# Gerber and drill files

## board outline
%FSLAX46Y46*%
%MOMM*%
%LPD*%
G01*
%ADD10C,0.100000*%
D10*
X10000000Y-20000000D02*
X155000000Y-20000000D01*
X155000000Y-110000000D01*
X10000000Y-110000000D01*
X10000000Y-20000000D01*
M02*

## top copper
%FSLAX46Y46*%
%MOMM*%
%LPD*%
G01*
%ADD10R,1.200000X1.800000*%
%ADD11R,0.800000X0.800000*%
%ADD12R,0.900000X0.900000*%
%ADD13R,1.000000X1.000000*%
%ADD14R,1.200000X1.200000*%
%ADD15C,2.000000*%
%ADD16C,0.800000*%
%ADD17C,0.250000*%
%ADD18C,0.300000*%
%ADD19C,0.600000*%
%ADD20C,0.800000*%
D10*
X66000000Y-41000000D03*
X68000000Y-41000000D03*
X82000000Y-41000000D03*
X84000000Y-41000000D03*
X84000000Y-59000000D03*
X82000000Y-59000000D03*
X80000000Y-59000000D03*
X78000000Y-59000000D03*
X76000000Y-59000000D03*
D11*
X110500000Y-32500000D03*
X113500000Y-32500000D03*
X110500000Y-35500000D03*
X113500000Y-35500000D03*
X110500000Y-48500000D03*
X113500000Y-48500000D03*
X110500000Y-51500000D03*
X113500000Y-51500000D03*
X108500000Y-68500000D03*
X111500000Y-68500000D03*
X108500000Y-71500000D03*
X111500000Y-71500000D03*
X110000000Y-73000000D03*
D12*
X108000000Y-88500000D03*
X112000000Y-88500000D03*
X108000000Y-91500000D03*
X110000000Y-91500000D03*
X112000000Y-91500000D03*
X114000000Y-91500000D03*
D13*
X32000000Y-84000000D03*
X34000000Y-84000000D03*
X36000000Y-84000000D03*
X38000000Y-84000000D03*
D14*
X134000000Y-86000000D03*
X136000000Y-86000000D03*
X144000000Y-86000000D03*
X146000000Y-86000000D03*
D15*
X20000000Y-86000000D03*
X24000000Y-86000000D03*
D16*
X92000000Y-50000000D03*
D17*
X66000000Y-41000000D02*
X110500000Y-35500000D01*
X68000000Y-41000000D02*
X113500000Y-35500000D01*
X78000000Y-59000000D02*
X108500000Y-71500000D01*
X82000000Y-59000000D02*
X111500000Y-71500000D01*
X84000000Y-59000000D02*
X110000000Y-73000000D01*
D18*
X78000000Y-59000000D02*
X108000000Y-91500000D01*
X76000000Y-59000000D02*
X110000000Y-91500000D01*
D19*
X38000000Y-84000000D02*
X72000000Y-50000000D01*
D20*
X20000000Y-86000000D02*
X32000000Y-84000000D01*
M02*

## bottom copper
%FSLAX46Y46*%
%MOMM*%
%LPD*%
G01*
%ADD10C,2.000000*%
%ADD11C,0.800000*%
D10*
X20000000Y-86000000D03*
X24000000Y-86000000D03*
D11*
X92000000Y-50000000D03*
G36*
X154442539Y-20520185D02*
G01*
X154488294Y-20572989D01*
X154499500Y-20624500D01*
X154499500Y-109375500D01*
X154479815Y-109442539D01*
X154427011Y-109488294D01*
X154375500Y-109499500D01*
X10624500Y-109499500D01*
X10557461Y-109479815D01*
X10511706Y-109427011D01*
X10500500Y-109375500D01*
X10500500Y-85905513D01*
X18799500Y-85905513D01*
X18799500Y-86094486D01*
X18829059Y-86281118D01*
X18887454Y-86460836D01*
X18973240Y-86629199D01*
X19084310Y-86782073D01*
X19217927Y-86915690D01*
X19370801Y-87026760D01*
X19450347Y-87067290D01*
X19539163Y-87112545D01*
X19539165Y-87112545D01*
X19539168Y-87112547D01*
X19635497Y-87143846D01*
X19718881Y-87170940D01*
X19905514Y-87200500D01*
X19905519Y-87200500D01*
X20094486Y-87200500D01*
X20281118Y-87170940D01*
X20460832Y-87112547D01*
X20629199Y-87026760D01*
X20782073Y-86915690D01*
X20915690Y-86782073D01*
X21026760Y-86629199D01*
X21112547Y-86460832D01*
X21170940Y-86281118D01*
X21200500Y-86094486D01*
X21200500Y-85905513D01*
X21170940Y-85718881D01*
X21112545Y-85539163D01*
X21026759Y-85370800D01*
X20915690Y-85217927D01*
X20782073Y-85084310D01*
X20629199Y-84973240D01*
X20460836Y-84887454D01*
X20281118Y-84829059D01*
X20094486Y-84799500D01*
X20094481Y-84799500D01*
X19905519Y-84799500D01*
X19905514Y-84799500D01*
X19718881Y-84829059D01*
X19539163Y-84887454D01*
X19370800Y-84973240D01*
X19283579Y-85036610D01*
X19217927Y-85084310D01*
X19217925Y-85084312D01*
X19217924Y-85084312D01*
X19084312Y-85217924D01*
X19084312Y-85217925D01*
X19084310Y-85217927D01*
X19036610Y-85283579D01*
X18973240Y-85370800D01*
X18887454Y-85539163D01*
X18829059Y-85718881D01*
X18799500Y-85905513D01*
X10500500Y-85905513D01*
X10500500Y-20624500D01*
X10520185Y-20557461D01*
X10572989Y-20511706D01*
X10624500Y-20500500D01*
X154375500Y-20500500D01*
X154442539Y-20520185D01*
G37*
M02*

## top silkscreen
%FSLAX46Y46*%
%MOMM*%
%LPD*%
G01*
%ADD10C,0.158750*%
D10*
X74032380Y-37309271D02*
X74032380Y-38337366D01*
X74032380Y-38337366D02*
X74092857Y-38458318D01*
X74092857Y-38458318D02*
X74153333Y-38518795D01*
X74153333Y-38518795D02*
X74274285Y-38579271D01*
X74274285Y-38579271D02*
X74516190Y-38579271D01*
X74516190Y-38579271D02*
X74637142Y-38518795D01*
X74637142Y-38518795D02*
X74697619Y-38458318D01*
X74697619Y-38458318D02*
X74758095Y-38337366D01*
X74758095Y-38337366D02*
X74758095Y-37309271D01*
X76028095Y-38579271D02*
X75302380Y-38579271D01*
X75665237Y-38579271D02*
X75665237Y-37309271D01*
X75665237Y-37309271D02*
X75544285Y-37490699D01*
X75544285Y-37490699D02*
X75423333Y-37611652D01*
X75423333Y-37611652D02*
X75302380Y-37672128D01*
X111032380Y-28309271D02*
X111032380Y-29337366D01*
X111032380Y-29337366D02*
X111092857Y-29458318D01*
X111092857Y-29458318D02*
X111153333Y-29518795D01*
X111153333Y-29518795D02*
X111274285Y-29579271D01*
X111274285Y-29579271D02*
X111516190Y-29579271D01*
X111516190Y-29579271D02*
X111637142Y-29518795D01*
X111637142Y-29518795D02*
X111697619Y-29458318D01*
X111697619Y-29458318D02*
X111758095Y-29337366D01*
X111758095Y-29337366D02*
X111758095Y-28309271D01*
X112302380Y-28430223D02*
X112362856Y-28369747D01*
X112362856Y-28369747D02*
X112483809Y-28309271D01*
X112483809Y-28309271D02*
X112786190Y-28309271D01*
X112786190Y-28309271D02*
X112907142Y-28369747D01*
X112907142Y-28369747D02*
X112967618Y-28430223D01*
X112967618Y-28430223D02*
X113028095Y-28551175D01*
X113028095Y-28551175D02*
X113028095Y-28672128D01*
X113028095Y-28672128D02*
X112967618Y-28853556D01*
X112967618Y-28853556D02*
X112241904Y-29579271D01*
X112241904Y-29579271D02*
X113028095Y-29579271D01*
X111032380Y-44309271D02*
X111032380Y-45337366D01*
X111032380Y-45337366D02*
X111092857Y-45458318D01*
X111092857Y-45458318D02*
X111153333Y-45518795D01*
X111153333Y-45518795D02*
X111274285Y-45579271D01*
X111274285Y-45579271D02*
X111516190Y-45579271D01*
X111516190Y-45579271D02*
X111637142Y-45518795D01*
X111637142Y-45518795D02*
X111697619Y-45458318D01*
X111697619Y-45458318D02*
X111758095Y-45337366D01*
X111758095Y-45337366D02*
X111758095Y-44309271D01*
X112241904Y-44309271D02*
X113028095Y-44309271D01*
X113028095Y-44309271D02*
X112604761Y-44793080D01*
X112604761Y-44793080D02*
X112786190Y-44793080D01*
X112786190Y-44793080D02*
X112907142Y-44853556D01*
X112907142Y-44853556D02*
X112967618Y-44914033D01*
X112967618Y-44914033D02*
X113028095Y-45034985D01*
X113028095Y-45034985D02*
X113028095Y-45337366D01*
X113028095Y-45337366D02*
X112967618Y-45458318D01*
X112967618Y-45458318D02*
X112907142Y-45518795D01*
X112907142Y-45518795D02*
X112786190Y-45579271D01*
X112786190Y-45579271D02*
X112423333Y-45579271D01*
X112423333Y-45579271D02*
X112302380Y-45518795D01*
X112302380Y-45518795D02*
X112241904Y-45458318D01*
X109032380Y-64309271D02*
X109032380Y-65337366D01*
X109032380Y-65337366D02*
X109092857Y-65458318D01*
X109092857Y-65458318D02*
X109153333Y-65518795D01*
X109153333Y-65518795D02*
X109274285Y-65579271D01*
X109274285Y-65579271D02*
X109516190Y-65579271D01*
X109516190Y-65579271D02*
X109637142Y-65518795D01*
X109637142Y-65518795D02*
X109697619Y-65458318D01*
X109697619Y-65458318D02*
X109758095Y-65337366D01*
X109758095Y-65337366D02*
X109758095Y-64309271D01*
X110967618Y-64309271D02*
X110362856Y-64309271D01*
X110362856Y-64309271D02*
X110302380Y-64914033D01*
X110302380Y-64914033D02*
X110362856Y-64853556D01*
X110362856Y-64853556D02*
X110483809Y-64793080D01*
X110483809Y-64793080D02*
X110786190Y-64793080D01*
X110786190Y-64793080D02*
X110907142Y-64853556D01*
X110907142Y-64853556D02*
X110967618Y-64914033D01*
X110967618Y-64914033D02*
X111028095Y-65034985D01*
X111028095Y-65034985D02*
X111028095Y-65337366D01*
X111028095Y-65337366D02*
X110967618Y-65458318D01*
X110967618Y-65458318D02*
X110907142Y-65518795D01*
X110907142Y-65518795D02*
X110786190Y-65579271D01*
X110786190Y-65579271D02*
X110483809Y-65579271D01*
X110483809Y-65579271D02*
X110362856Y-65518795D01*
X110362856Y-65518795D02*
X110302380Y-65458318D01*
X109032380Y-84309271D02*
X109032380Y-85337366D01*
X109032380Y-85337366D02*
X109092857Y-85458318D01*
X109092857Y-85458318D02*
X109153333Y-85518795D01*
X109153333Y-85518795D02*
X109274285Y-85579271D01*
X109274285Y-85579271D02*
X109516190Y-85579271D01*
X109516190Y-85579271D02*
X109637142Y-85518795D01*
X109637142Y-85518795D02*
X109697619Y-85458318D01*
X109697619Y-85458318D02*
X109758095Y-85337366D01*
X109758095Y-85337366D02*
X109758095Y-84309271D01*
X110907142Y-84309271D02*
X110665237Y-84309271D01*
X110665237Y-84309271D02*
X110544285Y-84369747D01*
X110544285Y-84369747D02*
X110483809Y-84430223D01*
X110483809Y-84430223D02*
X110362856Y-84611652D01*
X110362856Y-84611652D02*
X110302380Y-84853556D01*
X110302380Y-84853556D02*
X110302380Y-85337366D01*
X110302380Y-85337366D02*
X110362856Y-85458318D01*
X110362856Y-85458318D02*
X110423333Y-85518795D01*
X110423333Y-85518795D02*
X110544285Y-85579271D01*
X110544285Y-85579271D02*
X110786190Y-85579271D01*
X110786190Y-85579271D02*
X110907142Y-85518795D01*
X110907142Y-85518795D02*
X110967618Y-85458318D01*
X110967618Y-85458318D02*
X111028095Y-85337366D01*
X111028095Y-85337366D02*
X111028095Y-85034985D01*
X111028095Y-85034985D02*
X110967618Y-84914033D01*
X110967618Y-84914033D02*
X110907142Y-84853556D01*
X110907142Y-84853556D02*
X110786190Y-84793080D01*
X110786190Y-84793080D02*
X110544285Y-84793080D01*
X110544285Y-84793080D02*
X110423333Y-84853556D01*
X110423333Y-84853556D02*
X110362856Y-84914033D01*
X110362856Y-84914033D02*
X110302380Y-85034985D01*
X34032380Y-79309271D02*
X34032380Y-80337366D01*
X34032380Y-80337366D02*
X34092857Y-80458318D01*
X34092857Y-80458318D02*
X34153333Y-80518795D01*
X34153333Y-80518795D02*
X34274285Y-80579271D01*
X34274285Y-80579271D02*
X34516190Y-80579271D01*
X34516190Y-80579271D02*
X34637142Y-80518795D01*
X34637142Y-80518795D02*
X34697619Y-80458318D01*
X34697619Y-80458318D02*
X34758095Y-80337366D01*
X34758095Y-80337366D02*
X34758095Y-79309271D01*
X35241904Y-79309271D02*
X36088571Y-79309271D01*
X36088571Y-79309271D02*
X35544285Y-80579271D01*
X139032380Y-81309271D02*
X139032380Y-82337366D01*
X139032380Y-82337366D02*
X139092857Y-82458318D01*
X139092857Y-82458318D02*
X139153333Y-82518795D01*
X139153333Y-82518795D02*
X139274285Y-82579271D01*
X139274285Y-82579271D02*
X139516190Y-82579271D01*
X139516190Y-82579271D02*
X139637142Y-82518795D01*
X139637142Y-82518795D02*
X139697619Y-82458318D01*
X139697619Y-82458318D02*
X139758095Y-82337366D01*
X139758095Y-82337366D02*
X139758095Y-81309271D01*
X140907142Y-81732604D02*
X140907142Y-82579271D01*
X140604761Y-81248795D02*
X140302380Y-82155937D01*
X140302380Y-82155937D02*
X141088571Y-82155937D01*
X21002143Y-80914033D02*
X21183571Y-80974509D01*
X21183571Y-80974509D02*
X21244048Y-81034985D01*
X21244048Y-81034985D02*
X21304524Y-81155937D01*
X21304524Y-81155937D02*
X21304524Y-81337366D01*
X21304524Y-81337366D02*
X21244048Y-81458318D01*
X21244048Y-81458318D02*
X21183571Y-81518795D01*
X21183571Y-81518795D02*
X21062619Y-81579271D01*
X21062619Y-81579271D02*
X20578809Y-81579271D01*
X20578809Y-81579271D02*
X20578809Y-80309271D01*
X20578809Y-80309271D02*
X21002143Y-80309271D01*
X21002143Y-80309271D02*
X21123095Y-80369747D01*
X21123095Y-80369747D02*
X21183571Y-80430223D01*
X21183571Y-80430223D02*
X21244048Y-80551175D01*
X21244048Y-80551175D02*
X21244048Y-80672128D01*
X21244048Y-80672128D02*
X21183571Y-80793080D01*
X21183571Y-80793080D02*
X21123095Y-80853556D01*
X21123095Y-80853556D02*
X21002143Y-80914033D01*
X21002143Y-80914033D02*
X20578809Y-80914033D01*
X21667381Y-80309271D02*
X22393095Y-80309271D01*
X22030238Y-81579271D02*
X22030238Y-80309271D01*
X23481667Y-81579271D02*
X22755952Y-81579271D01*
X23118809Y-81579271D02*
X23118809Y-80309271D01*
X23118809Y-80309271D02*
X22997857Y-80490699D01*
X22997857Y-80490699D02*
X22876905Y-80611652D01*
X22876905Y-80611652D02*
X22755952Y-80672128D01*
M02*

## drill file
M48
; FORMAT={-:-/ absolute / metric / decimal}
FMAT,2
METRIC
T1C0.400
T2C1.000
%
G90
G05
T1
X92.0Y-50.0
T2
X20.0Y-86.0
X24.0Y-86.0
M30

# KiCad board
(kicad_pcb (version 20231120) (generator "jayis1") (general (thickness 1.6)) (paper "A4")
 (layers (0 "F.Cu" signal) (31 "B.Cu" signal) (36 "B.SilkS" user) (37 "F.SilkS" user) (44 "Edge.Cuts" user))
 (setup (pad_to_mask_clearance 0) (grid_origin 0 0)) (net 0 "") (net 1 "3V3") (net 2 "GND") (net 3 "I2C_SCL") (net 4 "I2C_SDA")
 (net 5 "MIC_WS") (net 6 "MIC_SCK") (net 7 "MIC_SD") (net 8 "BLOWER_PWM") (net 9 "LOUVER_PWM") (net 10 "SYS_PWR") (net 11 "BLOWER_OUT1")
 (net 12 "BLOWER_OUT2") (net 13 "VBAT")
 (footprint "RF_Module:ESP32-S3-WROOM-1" (layer "F.Cu") (at 75 50) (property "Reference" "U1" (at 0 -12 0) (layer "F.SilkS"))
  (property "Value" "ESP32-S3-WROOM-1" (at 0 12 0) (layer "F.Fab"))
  (pad "1" smd rect (at -9 -9) (size 1.2 1.8) (layers "F.Cu" "F.Mask") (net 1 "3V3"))
  (pad "2" smd rect (at -7 -9) (size 1.2 1.8) (layers "F.Cu" "F.Mask") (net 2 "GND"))
  (pad "5" smd rect (at 7 -9) (size 1.2 1.8) (layers "F.Cu" "F.Mask") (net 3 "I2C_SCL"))
  (pad "6" smd rect (at 9 -9) (size 1.2 1.8) (layers "F.Cu" "F.Mask") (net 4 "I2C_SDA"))
  (pad "7" smd rect (at 9 9) (size 1.2 1.8) (layers "F.Cu" "F.Mask") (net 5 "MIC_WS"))
  (pad "8" smd rect (at 7 9) (size 1.2 1.8) (layers "F.Cu" "F.Mask") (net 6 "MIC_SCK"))
  (pad "9" smd rect (at 5 9) (size 1.2 1.8) (layers "F.Cu" "F.Mask") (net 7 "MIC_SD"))
  (pad "10" smd rect (at 3 9) (size 1.2 1.8) (layers "F.Cu" "F.Mask") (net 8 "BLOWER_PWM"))
  (pad "11" smd rect (at 1 9) (size 1.2 1.8) (layers "F.Cu" "F.Mask") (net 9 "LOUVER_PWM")))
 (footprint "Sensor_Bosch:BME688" (layer "F.Cu") (at 112 34) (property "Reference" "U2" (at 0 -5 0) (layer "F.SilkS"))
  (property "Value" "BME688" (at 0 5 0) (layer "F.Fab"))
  (pad "1" smd rect (at -1.5 -1.5) (size 0.8 0.8) (layers "F.Cu" "F.Mask") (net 1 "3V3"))
  (pad "2" smd rect (at 1.5 -1.5) (size 0.8 0.8) (layers "F.Cu" "F.Mask") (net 2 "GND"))
  (pad "3" smd rect (at -1.5 1.5) (size 0.8 0.8) (layers "F.Cu" "F.Mask") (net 3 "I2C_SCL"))
  (pad "4" smd rect (at 1.5 1.5) (size 0.8 0.8) (layers "F.Cu" "F.Mask") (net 4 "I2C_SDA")))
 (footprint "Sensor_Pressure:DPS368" (layer "F.Cu") (at 112 50) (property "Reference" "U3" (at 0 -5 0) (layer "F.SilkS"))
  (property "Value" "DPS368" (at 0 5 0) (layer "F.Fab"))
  (pad "1" smd rect (at -1.5 -1.5) (size 0.8 0.8) (layers "F.Cu" "F.Mask") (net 1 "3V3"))
  (pad "2" smd rect (at 1.5 -1.5) (size 0.8 0.8) (layers "F.Cu" "F.Mask") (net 2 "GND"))
  (pad "3" smd rect (at -1.5 1.5) (size 0.8 0.8) (layers "F.Cu" "F.Mask") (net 3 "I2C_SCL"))
  (pad "4" smd rect (at 1.5 1.5) (size 0.8 0.8) (layers "F.Cu" "F.Mask") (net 4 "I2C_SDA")))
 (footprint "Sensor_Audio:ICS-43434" (layer "F.Cu") (at 110 70) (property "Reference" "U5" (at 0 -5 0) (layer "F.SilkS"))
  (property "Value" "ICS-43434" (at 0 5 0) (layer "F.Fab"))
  (pad "1" smd rect (at -1.5 -1.5) (size 0.8 0.8) (layers "F.Cu" "F.Mask") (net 1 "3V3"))
  (pad "2" smd rect (at 1.5 -1.5) (size 0.8 0.8) (layers "F.Cu" "F.Mask") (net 2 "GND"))
  (pad "3" smd rect (at -1.5 1.5) (size 0.8 0.8) (layers "F.Cu" "F.Mask") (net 7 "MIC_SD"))
  (pad "4" smd rect (at 1.5 1.5) (size 0.8 0.8) (layers "F.Cu" "F.Mask") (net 6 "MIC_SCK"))
  (pad "5" smd rect (at 0 3.0) (size 0.8 0.8) (layers "F.Cu" "F.Mask") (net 5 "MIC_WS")))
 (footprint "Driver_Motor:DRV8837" (layer "F.Cu") (at 110 90) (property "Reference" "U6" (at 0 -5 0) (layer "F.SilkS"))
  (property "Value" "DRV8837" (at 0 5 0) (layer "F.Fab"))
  (pad "1" smd rect (at -2 -1.5) (size 0.9 0.9) (layers "F.Cu" "F.Mask") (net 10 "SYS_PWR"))
  (pad "2" smd rect (at 2 -1.5) (size 0.9 0.9) (layers "F.Cu" "F.Mask") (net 2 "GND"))
  (pad "3" smd rect (at -2 1.5) (size 0.9 0.9) (layers "F.Cu" "F.Mask") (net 8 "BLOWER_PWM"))
  (pad "4" smd rect (at 0 1.5) (size 0.9 0.9) (layers "F.Cu" "F.Mask") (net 9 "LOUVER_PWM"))
  (pad "5" smd rect (at 2 1.5) (size 0.9 0.9) (layers "F.Cu" "F.Mask") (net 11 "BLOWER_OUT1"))
  (pad "6" smd rect (at 4 1.5) (size 0.9 0.9) (layers "F.Cu" "F.Mask") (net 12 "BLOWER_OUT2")))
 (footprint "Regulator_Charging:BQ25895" (layer "F.Cu") (at 35 86) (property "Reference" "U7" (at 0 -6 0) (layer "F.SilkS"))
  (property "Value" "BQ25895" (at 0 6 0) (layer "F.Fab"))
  (pad "1" smd rect (at -3 -2) (size 1 1) (layers "F.Cu" "F.Mask") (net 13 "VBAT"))
  (pad "2" smd rect (at -1 -2) (size 1 1) (layers "F.Cu" "F.Mask") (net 13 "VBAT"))
  (pad "3" smd rect (at 1 -2) (size 1 1) (layers "F.Cu" "F.Mask") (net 2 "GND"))
  (pad "4" smd rect (at 3 -2) (size 1 1) (layers "F.Cu" "F.Mask") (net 10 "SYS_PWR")))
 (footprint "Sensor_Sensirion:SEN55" (layer "F.Cu") (at 140 90) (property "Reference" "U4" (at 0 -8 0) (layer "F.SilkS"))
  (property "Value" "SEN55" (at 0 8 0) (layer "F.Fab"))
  (pad "1" smd rect (at -6 -4) (size 1.2 1.2) (layers "F.Cu" "F.Mask") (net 10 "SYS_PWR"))
  (pad "2" smd rect (at -4 -4) (size 1.2 1.2) (layers "F.Cu" "F.Mask") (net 2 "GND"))
  (pad "3" smd rect (at 4 -4) (size 1.2 1.2) (layers "F.Cu" "F.Mask") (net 3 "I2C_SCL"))
  (pad "4" smd rect (at 6 -4) (size 1.2 1.2) (layers "F.Cu" "F.Mask") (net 4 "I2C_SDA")))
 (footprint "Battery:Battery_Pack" (layer "F.Cu") (at 22 86) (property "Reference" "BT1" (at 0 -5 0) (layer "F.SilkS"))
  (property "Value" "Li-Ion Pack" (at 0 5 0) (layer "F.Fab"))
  (pad "1" thru_hole circle (at -2 0) (size 2 2) (drill 1.0) (layers *.Cu *.Mask) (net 13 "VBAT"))
  (pad "2" thru_hole circle (at 2 0) (size 2 2) (drill 1.0) (layers *.Cu *.Mask) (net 2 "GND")))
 (gr_rect (start 10 20) (end 155 110) (stroke (width 0.1) (type default)) (fill none) (layer "Edge.Cuts"))
 (segment (start 66 41) (end 110.5 35.5) (width 0.25) (layer "F.Cu") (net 3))
 (segment (start 68 41) (end 113.5 35.5) (width 0.25) (layer "F.Cu") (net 4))
 (segment (start 78 59) (end 108.5 71.5) (width 0.25) (layer "F.Cu") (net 7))
 (segment (start 82 59) (end 111.5 71.5) (width 0.25) (layer "F.Cu") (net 6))
 (segment (start 84 59) (end 110 73.0) (width 0.25) (layer "F.Cu") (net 5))
 (segment (start 78 59) (end 108 91.5) (width 0.30) (layer "F.Cu") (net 8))
 (segment (start 76 59) (end 110 91.5) (width 0.30) (layer "F.Cu") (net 9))
 (segment (start 38 84) (end 72 50) (width 0.60) (layer "F.Cu") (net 10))
 (segment (start 20 86) (end 32 84) (width 0.80) (layer "F.Cu") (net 13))
 (via (at 92 50) (size 0.8) (drill 0.4) (layers "F.Cu" "B.Cu") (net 2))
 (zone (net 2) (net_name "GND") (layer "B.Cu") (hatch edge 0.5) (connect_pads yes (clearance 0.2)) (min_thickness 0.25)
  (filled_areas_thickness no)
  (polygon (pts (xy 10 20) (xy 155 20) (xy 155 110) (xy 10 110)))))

